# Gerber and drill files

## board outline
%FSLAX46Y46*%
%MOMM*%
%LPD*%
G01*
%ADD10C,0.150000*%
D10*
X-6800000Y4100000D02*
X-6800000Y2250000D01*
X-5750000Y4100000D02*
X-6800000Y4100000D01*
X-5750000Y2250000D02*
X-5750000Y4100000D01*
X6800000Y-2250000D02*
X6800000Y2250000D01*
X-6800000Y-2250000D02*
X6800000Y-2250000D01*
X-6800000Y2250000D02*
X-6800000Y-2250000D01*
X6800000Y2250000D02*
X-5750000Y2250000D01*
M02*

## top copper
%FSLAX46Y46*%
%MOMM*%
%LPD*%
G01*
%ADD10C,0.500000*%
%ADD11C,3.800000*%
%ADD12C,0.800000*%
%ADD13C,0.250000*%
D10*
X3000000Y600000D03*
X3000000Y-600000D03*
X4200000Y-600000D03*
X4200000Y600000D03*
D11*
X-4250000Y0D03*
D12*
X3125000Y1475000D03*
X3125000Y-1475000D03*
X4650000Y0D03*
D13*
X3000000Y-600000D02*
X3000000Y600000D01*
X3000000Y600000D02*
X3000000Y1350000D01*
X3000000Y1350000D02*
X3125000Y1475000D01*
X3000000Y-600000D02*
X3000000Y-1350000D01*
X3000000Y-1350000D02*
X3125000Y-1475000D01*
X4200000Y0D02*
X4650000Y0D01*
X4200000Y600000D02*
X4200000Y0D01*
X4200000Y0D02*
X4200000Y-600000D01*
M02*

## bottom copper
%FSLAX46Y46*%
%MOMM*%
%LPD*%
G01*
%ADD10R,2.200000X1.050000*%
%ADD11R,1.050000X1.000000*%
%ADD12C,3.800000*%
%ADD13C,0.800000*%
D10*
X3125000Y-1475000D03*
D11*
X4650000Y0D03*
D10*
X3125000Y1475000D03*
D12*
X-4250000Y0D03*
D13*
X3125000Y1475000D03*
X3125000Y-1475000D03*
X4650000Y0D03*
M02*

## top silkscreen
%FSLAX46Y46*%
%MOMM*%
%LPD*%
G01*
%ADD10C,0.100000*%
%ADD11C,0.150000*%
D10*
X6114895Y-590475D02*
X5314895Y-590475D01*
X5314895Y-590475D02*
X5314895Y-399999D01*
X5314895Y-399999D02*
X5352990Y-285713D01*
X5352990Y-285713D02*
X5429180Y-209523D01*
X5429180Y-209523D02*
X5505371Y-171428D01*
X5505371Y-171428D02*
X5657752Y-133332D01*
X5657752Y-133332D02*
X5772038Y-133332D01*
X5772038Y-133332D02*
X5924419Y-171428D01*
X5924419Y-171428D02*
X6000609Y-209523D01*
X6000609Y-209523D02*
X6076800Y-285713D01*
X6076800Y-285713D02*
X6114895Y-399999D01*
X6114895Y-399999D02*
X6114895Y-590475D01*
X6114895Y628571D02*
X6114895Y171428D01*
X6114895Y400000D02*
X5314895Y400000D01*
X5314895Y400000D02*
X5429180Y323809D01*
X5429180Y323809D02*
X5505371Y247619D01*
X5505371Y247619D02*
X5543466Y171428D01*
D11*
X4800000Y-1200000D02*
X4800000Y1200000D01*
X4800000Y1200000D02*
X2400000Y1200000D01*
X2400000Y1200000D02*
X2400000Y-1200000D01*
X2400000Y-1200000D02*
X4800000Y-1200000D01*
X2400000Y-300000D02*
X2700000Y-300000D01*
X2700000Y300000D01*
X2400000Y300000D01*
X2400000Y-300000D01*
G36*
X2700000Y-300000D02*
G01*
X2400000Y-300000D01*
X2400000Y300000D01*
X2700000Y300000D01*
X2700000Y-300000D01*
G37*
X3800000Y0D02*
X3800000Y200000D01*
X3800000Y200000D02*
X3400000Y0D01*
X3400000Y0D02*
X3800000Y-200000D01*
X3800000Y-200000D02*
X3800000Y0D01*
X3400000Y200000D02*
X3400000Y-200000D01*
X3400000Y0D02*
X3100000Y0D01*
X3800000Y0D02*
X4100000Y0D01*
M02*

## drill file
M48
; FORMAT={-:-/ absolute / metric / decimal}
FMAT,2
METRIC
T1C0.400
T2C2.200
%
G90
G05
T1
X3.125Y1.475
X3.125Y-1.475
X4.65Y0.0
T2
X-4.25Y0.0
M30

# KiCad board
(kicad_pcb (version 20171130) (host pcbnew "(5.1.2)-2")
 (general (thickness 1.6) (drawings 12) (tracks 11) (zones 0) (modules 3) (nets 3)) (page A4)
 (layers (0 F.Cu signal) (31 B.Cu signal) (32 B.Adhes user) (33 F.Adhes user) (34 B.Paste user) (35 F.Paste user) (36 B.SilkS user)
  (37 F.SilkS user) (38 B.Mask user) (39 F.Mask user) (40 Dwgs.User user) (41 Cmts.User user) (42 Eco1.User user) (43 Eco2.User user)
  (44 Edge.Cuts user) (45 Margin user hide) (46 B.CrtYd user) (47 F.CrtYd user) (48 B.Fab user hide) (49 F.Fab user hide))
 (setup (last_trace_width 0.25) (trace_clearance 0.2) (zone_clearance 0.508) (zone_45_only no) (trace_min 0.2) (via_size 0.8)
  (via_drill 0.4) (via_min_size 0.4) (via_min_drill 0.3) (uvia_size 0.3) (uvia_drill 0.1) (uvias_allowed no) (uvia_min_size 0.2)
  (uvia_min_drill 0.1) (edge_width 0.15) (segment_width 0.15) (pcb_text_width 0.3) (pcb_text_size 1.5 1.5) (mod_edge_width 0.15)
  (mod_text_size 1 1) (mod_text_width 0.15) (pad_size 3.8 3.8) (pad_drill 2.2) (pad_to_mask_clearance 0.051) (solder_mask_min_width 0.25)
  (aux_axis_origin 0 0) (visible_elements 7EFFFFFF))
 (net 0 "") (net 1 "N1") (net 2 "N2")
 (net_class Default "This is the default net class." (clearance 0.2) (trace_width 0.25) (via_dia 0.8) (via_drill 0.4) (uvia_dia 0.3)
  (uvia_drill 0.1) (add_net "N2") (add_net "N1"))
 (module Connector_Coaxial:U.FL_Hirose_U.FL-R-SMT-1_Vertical (layer B.Cu) (at 3.6 0 180)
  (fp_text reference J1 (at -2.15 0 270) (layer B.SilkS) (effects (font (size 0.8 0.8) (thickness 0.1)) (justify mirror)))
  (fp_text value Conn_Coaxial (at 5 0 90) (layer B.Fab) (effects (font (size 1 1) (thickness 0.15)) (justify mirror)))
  (pad 2 smd rect (at 0.475 -1.475 180) (size 2.2 1.05) (layers B.Cu B.Paste B.Mask) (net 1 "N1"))
  (pad 1 smd rect (at -1.05 0 180) (size 1.05 1) (layers B.Cu B.Paste B.Mask) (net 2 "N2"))
  (pad 2 smd rect (at 0.475 1.475 180) (size 2.2 1.05) (layers B.Cu B.Paste B.Mask) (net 1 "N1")))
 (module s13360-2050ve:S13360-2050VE (layer F.Cu) (at 3.6 0 270)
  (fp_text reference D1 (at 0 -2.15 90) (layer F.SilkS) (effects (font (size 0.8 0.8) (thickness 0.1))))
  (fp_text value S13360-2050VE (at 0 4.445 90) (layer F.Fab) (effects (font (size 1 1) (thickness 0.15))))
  (fp_line (start 1.2 -1.2) (end -1.2 -1.2) (layer F.SilkS) (width 0.15))
  (fp_line (start -1.2 -1.2) (end -1.2 1.2) (layer F.SilkS) (width 0.15))
  (fp_line (start -1.2 1.2) (end 1.2 1.2) (layer F.SilkS) (width 0.15))
  (fp_line (start 1.2 1.2) (end 1.2 -1.2) (layer F.SilkS) (width 0.15))
  (fp_poly (pts (xy 0.3 1.2) (xy 0.3 0.9) (xy -0.3 0.9) (xy -0.3 1.2)) (layer F.SilkS) (width 0.15))
  (fp_line (start 0 -0.2) (end -0.2 -0.2) (layer F.SilkS) (width 0.15))
  (fp_line (start -0.2 -0.2) (end 0 0.2) (layer F.SilkS) (width 0.15))
  (fp_line (start 0 0.2) (end 0.2 -0.2) (layer F.SilkS) (width 0.15))
  (fp_line (start 0.2 -0.2) (end 0 -0.2) (layer F.SilkS) (width 0.15))
  (fp_line (start -0.2 0.2) (end 0.2 0.2) (layer F.SilkS) (width 0.15))
  (fp_line (start 0 0.2) (end 0 0.5) (layer F.SilkS) (width 0.15))
  (fp_line (start 0 -0.2) (end 0 -0.5) (layer F.SilkS) (width 0.15))
  (pad 2 smd circle (at -0.6 0.6 270) (size 0.5 0.5) (layers F.Cu F.Paste F.Mask) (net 1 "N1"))
  (pad 2 smd circle (at 0.6 0.6 270) (size 0.5 0.5) (layers F.Cu F.Paste F.Mask) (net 1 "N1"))
  (pad 1 smd circle (at 0.6 -0.6 270) (size 0.5 0.5) (layers F.Cu F.Paste F.Mask) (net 2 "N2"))
  (pad 1 smd circle (at -0.6 -0.6 270) (size 0.5 0.5) (layers F.Cu F.Paste F.Mask) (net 2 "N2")))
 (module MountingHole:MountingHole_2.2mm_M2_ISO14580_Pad (layer F.Cu) (at -4.25 0)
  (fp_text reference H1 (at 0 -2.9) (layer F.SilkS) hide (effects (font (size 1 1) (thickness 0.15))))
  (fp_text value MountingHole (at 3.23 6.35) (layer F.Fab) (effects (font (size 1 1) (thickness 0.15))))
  (pad 1 thru_hole circle (at 0 0) (size 3.8 3.8) (drill 2.2) (layers *.Cu *.Mask)))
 (gr_line (start -6.8 -4.1) (end -6.8 -2.25) (layer Edge.Cuts) (width 0.15))
 (gr_line (start -5.75 -4.1) (end -6.8 -4.1) (layer Edge.Cuts) (width 0.15))
 (gr_line (start -5.75 -2.25) (end -5.75 -4.1) (layer Edge.Cuts) (width 0.15))
 (gr_line (start 6.8 2.25) (end 6.8 -2.25) (layer Edge.Cuts) (width 0.15))
 (gr_line (start -6.8 2.25) (end 6.8 2.25) (layer Edge.Cuts) (width 0.15))
 (gr_line (start -6.8 -2.25) (end -6.8 2.25) (layer Edge.Cuts) (width 0.15))
 (gr_line (start 6.8 -2.25) (end -5.75 -2.25) (layer Edge.Cuts) (width 0.15))
 (segment (start 3 0.6) (end 3 -0.6) (width 0.25) (layer F.Cu) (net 1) (status 30))
 (via (at 3.125 -1.475) (size 0.8) (drill 0.4) (layers F.Cu B.Cu) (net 1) (status 30))
 (segment (start 3 -0.6) (end 3 -1.35) (width 0.25) (layer F.Cu) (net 1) (status 10))
 (segment (start 3 -1.35) (end 3.125 -1.475) (width 0.25) (layer F.Cu) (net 1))
 (via (at 3.125 1.475) (size 0.8) (drill 0.4) (layers F.Cu B.Cu) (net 1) (status 30))
 (segment (start 3 0.6) (end 3 1.35) (width 0.25) (layer F.Cu) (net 1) (status 10))
 (segment (start 3 1.35) (end 3.125 1.475) (width 0.25) (layer F.Cu) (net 1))
 (via (at 4.65 0) (size 0.8) (drill 0.4) (layers F.Cu B.Cu) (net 2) (status 30))
 (segment (start 4.2 0) (end 4.65 0) (width 0.25) (layer F.Cu) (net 2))
 (segment (start 4.2 -0.6) (end 4.2 0) (width 0.25) (layer F.Cu) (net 2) (status 10))
 (segment (start 4.2 0) (end 4.2 0.6) (width 0.25) (layer F.Cu) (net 2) (status 20)))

